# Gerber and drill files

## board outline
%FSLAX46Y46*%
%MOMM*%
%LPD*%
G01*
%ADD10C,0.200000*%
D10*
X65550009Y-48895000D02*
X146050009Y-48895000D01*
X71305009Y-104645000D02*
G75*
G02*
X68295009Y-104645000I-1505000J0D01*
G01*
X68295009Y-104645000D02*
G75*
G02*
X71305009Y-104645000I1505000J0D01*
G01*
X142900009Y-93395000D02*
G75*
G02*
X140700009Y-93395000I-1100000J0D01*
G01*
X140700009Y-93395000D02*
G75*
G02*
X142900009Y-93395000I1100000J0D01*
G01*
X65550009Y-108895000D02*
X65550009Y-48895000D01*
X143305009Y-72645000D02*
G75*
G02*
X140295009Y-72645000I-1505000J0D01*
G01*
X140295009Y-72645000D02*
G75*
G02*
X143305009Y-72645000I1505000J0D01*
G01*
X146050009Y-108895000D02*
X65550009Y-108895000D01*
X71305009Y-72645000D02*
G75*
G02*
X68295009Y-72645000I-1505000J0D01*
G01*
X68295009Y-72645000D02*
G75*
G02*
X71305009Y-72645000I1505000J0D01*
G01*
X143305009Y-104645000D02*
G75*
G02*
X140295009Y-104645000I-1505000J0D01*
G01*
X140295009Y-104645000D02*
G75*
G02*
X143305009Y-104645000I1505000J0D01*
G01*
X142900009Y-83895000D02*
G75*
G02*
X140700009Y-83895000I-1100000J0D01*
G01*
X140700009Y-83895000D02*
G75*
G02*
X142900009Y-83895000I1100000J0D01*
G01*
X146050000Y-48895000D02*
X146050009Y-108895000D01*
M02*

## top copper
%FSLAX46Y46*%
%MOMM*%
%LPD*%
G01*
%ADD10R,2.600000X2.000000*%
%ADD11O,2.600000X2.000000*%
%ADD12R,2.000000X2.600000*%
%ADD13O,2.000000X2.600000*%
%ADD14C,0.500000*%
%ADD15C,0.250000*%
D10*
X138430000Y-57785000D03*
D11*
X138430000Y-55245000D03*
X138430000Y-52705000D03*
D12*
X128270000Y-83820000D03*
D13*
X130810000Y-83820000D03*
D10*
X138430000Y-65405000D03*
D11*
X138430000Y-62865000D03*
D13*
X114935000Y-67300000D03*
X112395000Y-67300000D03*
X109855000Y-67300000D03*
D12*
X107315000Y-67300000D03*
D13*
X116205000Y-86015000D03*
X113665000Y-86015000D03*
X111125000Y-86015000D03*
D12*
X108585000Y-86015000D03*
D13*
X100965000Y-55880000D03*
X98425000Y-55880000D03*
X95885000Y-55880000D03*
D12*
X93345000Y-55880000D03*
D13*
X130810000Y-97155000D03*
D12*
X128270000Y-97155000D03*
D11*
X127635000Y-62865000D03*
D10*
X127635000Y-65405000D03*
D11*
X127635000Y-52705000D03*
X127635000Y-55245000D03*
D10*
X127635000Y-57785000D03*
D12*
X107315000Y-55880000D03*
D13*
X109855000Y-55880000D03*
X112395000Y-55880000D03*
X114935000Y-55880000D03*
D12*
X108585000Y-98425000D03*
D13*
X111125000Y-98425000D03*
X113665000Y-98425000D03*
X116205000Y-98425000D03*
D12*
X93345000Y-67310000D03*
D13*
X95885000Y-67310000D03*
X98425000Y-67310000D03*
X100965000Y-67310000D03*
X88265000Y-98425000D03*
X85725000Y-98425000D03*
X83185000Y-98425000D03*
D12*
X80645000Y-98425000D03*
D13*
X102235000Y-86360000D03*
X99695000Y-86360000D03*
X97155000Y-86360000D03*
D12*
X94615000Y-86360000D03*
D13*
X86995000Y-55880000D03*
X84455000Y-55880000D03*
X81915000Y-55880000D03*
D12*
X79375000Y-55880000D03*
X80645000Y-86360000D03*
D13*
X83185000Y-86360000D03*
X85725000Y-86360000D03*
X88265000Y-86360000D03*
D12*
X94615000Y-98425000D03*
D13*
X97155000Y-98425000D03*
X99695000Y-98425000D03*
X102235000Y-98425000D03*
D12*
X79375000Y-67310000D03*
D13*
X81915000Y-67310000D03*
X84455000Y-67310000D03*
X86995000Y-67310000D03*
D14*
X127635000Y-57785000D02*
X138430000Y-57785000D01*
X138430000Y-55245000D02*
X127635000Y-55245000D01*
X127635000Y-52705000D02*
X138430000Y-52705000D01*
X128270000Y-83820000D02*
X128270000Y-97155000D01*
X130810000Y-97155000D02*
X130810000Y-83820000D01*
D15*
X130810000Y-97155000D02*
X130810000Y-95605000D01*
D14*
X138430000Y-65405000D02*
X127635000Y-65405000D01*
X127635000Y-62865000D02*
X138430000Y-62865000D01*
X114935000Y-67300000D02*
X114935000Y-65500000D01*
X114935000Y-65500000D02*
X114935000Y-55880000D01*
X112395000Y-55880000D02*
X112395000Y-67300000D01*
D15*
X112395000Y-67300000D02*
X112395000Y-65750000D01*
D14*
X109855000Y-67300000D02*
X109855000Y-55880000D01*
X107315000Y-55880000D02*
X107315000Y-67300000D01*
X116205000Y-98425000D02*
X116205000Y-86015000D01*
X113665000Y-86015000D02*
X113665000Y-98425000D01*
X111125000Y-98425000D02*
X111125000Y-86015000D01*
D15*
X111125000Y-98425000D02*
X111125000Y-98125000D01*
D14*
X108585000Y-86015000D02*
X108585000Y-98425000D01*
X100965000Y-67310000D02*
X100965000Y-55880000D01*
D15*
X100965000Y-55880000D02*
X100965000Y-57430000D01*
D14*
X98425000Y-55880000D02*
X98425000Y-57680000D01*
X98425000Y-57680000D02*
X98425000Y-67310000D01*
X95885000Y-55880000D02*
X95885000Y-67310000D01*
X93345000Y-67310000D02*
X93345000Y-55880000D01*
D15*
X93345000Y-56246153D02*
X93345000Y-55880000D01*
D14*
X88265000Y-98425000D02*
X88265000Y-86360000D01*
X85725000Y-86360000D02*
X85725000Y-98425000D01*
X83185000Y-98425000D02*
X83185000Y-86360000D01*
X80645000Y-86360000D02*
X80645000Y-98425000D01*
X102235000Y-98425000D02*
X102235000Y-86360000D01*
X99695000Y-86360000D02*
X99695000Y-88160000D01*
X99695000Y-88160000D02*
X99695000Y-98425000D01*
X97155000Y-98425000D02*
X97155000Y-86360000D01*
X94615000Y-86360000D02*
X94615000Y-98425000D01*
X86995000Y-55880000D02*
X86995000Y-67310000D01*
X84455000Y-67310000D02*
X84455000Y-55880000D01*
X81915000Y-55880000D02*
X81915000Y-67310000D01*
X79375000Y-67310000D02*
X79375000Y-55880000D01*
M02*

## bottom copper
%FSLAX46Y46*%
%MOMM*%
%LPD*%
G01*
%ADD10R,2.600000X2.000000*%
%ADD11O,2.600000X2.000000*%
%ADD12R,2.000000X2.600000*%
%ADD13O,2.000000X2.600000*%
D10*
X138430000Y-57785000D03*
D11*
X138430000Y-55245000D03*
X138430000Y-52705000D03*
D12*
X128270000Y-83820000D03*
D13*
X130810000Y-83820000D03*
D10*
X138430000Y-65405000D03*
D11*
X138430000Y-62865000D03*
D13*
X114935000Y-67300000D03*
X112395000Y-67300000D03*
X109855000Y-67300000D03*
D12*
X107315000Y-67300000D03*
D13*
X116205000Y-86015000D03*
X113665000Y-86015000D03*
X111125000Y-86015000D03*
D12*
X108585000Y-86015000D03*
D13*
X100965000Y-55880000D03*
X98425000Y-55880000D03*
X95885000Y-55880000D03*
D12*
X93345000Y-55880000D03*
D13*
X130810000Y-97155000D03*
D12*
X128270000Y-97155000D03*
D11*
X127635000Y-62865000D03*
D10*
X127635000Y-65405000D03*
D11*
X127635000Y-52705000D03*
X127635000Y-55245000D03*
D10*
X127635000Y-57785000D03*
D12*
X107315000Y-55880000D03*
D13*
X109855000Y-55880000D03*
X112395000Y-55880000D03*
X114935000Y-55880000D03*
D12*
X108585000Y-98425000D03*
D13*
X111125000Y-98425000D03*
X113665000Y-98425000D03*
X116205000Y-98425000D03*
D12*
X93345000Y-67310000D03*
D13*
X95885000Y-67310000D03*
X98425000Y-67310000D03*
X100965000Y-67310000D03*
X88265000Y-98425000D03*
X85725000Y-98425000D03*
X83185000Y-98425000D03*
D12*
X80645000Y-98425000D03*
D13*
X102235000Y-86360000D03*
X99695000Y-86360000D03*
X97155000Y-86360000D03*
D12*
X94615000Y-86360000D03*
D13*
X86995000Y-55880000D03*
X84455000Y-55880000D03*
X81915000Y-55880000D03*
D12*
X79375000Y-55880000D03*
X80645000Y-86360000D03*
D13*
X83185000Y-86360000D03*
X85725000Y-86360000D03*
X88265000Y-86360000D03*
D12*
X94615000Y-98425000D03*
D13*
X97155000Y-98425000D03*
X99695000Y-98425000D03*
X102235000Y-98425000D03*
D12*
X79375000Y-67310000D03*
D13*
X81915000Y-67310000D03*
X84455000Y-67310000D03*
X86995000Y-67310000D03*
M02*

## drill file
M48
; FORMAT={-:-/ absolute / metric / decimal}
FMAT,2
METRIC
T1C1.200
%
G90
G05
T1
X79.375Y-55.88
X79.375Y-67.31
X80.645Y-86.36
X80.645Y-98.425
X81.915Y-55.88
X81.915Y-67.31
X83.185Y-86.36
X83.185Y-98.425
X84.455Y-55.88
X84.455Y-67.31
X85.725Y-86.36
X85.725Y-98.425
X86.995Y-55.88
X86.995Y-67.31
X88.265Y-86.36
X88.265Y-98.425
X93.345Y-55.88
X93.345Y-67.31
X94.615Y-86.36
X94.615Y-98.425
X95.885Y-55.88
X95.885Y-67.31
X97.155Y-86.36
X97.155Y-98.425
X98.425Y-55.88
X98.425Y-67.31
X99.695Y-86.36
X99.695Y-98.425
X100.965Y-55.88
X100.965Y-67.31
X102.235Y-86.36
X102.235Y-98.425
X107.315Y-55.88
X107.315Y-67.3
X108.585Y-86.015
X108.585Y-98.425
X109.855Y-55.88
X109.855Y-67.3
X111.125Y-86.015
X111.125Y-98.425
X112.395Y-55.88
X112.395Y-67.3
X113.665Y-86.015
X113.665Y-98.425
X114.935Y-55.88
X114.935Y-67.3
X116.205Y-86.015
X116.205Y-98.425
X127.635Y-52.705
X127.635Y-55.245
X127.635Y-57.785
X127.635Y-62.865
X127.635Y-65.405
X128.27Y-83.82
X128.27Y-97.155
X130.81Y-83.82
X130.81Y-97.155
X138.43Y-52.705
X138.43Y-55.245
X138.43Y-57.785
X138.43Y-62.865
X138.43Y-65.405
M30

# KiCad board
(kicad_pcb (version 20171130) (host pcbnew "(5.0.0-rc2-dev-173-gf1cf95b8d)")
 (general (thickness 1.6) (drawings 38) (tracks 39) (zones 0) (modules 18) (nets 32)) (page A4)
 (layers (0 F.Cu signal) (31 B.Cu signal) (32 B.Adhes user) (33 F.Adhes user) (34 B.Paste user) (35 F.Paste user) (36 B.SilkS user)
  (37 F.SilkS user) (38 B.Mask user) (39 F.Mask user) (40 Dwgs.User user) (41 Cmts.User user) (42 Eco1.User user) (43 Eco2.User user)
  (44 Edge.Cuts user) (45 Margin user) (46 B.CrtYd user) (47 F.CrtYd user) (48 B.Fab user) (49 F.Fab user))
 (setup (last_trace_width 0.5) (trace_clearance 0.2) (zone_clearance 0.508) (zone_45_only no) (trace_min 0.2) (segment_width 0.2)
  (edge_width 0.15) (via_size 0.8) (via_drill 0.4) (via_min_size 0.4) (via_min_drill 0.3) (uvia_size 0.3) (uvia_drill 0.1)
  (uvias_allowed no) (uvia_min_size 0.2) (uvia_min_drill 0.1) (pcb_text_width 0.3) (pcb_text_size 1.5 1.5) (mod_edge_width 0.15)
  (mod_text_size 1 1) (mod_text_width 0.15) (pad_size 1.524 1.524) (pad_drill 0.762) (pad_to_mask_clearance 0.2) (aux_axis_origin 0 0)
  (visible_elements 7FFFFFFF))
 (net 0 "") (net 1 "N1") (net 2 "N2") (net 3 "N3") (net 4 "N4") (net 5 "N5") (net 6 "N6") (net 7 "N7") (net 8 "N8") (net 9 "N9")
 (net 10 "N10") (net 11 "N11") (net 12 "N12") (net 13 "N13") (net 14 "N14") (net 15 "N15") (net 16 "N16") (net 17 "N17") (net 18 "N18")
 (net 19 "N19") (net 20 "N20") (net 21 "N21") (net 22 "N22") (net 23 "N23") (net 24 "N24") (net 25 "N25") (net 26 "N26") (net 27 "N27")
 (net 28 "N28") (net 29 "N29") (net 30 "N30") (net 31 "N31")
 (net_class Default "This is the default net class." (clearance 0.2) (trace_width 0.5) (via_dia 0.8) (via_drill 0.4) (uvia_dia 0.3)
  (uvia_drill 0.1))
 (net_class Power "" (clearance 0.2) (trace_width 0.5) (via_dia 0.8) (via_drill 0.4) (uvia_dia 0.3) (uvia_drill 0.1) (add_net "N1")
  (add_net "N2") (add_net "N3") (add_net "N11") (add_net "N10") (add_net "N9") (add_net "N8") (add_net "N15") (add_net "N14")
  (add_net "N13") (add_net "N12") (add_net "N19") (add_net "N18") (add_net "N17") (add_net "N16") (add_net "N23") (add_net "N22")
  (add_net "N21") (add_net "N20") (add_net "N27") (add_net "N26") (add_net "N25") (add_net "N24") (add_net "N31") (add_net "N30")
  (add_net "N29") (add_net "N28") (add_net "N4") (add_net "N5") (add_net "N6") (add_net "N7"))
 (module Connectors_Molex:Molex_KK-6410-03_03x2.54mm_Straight (layer F.Cu) (at 138.43 57.785 90)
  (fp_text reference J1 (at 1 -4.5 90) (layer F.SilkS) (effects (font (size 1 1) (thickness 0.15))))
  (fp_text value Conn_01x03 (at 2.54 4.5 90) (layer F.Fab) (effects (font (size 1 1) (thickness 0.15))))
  (pad 1 thru_hole rect (at 0 0 90) (size 2 2.6) (drill 1.2) (layers *.Cu *.Mask) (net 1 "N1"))
  (pad 2 thru_hole oval (at 2.54 0 90) (size 2 2.6) (drill 1.2) (layers *.Cu *.Mask) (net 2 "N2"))
  (pad 3 thru_hole oval (at 5.08 0 90) (size 2 2.6) (drill 1.2) (layers *.Cu *.Mask) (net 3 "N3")))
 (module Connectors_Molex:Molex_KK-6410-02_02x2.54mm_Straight (layer F.Cu) (at 128.27 83.82)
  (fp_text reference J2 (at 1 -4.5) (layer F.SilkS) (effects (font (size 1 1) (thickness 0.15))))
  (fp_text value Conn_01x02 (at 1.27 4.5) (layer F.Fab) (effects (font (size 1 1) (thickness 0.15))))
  (pad 1 thru_hole rect (at 0 0) (size 2 2.6) (drill 1.2) (layers *.Cu *.Mask) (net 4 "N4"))
  (pad 2 thru_hole oval (at 2.54 0) (size 2 2.6) (drill 1.2) (layers *.Cu *.Mask) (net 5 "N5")))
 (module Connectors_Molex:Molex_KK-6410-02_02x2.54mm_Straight (layer F.Cu) (at 138.43 65.405 90)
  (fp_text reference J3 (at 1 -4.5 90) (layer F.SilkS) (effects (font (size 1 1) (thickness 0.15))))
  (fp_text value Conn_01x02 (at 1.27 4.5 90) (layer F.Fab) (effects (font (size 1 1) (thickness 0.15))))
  (pad 1 thru_hole rect (at 0 0 90) (size 2 2.6) (drill 1.2) (layers *.Cu *.Mask) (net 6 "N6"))
  (pad 2 thru_hole oval (at 2.54 0 90) (size 2 2.6) (drill 1.2) (layers *.Cu *.Mask) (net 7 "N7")))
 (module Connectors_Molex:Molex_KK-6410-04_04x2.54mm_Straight (layer F.Cu) (at 107.315 67.3)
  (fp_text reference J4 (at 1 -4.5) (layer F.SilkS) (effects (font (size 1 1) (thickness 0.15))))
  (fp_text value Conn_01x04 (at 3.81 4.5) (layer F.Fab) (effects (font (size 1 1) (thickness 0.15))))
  (pad 4 thru_hole oval (at 7.62 0) (size 2 2.6) (drill 1.2) (layers *.Cu *.Mask) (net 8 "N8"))
  (pad 3 thru_hole oval (at 5.08 0) (size 2 2.6) (drill 1.2) (layers *.Cu *.Mask) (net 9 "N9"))
  (pad 2 thru_hole oval (at 2.54 0) (size 2 2.6) (drill 1.2) (layers *.Cu *.Mask) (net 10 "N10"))
  (pad 1 thru_hole rect (at 0 0) (size 2 2.6) (drill 1.2) (layers *.Cu *.Mask) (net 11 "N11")))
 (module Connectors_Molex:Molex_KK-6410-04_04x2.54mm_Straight (layer F.Cu) (at 108.585 86.015)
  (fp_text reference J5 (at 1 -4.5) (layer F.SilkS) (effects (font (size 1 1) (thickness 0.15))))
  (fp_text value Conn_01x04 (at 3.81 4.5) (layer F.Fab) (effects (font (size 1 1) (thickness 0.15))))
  (pad 4 thru_hole oval (at 7.62 0) (size 2 2.6) (drill 1.2) (layers *.Cu *.Mask) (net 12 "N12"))
  (pad 3 thru_hole oval (at 5.08 0) (size 2 2.6) (drill 1.2) (layers *.Cu *.Mask) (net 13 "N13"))
  (pad 2 thru_hole oval (at 2.54 0) (size 2 2.6) (drill 1.2) (layers *.Cu *.Mask) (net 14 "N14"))
  (pad 1 thru_hole rect (at 0 0) (size 2 2.6) (drill 1.2) (layers *.Cu *.Mask) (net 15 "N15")))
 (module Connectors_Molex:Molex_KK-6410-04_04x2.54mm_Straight (layer F.Cu) (at 93.345 55.88)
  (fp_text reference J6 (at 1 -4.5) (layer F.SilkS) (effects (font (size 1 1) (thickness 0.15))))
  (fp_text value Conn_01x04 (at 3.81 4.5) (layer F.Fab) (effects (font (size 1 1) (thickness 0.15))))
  (pad 4 thru_hole oval (at 7.62 0) (size 2 2.6) (drill 1.2) (layers *.Cu *.Mask) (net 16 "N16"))
  (pad 3 thru_hole oval (at 5.08 0) (size 2 2.6) (drill 1.2) (layers *.Cu *.Mask) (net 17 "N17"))
  (pad 2 thru_hole oval (at 2.54 0) (size 2 2.6) (drill 1.2) (layers *.Cu *.Mask) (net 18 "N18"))
  (pad 1 thru_hole rect (at 0 0) (size 2 2.6) (drill 1.2) (layers *.Cu *.Mask) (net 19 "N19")))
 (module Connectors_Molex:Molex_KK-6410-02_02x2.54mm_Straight (layer F.Cu) (at 128.27 97.155)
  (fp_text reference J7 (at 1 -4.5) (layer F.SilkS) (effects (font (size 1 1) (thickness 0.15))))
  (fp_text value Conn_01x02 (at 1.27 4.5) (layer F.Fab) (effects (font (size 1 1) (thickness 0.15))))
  (pad 2 thru_hole oval (at 2.54 0) (size 2 2.6) (drill 1.2) (layers *.Cu *.Mask) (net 5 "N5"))
  (pad 1 thru_hole rect (at 0 0) (size 2 2.6) (drill 1.2) (layers *.Cu *.Mask) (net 4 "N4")))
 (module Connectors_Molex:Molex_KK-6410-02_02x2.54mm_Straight (layer F.Cu) (at 127.635 65.405 90)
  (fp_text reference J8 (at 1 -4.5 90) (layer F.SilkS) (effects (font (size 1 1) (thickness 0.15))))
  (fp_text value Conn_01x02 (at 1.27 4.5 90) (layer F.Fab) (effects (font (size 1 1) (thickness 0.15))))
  (pad 2 thru_hole oval (at 2.54 0 90) (size 2 2.6) (drill 1.2) (layers *.Cu *.Mask) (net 7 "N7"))
  (pad 1 thru_hole rect (at 0 0 90) (size 2 2.6) (drill 1.2) (layers *.Cu *.Mask) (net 6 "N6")))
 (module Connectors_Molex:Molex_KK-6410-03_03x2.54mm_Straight (layer F.Cu) (at 127.635 57.785 90)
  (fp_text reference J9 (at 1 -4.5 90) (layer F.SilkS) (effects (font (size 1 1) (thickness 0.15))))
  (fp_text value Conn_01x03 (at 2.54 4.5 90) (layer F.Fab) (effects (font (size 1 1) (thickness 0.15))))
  (pad 3 thru_hole oval (at 5.08 0 90) (size 2 2.6) (drill 1.2) (layers *.Cu *.Mask) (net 3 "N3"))
  (pad 2 thru_hole oval (at 2.54 0 90) (size 2 2.6) (drill 1.2) (layers *.Cu *.Mask) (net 2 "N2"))
  (pad 1 thru_hole rect (at 0 0 90) (size 2 2.6) (drill 1.2) (layers *.Cu *.Mask) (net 1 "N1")))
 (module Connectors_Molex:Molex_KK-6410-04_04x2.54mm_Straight (layer F.Cu) (at 107.315 55.88)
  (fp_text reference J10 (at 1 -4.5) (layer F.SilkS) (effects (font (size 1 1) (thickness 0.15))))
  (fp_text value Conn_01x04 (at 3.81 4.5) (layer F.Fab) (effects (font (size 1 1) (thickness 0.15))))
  (pad 1 thru_hole rect (at 0 0) (size 2 2.6) (drill 1.2) (layers *.Cu *.Mask) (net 11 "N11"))
  (pad 2 thru_hole oval (at 2.54 0) (size 2 2.6) (drill 1.2) (layers *.Cu *.Mask) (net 10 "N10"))
  (pad 3 thru_hole oval (at 5.08 0) (size 2 2.6) (drill 1.2) (layers *.Cu *.Mask) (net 9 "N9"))
  (pad 4 thru_hole oval (at 7.62 0) (size 2 2.6) (drill 1.2) (layers *.Cu *.Mask) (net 8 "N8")))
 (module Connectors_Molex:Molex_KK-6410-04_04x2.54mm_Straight (layer F.Cu) (at 108.585 98.425)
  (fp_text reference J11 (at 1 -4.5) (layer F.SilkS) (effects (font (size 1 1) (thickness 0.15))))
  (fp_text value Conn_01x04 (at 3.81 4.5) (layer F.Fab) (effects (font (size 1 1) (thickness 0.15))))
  (pad 1 thru_hole rect (at 0 0) (size 2 2.6) (drill 1.2) (layers *.Cu *.Mask) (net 15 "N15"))
  (pad 2 thru_hole oval (at 2.54 0) (size 2 2.6) (drill 1.2) (layers *.Cu *.Mask) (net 14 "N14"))
  (pad 3 thru_hole oval (at 5.08 0) (size 2 2.6) (drill 1.2) (layers *.Cu *.Mask) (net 13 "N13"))
  (pad 4 thru_hole oval (at 7.62 0) (size 2 2.6) (drill 1.2) (layers *.Cu *.Mask) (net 12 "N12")))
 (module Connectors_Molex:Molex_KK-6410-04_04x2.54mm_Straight (layer F.Cu) (at 93.345 67.31)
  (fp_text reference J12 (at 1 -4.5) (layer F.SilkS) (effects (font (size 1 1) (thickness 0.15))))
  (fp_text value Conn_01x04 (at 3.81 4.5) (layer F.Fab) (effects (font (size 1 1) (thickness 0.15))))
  (pad 1 thru_hole rect (at 0 0) (size 2 2.6) (drill 1.2) (layers *.Cu *.Mask) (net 19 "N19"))
  (pad 2 thru_hole oval (at 2.54 0) (size 2 2.6) (drill 1.2) (layers *.Cu *.Mask) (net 18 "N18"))
  (pad 3 thru_hole oval (at 5.08 0) (size 2 2.6) (drill 1.2) (layers *.Cu *.Mask) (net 17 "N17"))
  (pad 4 thru_hole oval (at 7.62 0) (size 2 2.6) (drill 1.2) (layers *.Cu *.Mask) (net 16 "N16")))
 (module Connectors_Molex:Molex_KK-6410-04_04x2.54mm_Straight (layer F.Cu) (at 80.645 98.425)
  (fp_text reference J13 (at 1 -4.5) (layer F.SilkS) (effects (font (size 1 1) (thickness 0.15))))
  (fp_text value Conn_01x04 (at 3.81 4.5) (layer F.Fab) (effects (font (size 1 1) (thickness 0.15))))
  (pad 4 thru_hole oval (at 7.62 0) (size 2 2.6) (drill 1.2) (layers *.Cu *.Mask) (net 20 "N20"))
  (pad 3 thru_hole oval (at 5.08 0) (size 2 2.6) (drill 1.2) (layers *.Cu *.Mask) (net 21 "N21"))
  (pad 2 thru_hole oval (at 2.54 0) (size 2 2.6) (drill 1.2) (layers *.Cu *.Mask) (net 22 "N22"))
  (pad 1 thru_hole rect (at 0 0) (size 2 2.6) (drill 1.2) (layers *.Cu *.Mask) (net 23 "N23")))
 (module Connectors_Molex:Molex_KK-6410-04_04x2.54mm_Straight (layer F.Cu) (at 94.615 86.36)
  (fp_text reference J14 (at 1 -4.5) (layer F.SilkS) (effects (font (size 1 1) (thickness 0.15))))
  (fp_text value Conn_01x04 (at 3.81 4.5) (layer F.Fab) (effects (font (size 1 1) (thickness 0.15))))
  (pad 4 thru_hole oval (at 7.62 0) (size 2 2.6) (drill 1.2) (layers *.Cu *.Mask) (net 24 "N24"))
  (pad 3 thru_hole oval (at 5.08 0) (size 2 2.6) (drill 1.2) (layers *.Cu *.Mask) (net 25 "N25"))
  (pad 2 thru_hole oval (at 2.54 0) (size 2 2.6) (drill 1.2) (layers *.Cu *.Mask) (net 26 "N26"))
  (pad 1 thru_hole rect (at 0 0) (size 2 2.6) (drill 1.2) (layers *.Cu *.Mask) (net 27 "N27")))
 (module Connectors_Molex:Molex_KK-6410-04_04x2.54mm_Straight (layer F.Cu) (at 79.375 55.88)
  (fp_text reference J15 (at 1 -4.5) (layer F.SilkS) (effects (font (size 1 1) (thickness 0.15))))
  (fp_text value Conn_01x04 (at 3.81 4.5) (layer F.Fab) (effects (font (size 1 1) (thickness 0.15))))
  (pad 4 thru_hole oval (at 7.62 0) (size 2 2.6) (drill 1.2) (layers *.Cu *.Mask) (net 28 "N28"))
  (pad 3 thru_hole oval (at 5.08 0) (size 2 2.6) (drill 1.2) (layers *.Cu *.Mask) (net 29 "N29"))
  (pad 2 thru_hole oval (at 2.54 0) (size 2 2.6) (drill 1.2) (layers *.Cu *.Mask) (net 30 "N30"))
  (pad 1 thru_hole rect (at 0 0) (size 2 2.6) (drill 1.2) (layers *.Cu *.Mask) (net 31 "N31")))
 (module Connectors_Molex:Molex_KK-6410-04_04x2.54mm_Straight (layer F.Cu) (at 80.645 86.36)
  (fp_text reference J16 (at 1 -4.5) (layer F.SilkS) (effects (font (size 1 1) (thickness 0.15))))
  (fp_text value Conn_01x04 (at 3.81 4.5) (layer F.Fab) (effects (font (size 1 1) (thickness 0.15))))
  (pad 1 thru_hole rect (at 0 0) (size 2 2.6) (drill 1.2) (layers *.Cu *.Mask) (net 23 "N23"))
  (pad 2 thru_hole oval (at 2.54 0) (size 2 2.6) (drill 1.2) (layers *.Cu *.Mask) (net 22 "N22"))
  (pad 3 thru_hole oval (at 5.08 0) (size 2 2.6) (drill 1.2) (layers *.Cu *.Mask) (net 21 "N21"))
  (pad 4 thru_hole oval (at 7.62 0) (size 2 2.6) (drill 1.2) (layers *.Cu *.Mask) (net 20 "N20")))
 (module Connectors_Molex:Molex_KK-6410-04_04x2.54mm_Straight (layer F.Cu) (at 94.615 98.425)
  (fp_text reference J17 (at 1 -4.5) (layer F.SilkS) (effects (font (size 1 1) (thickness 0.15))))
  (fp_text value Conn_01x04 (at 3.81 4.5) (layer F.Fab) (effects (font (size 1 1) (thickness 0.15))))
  (pad 1 thru_hole rect (at 0 0) (size 2 2.6) (drill 1.2) (layers *.Cu *.Mask) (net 27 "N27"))
  (pad 2 thru_hole oval (at 2.54 0) (size 2 2.6) (drill 1.2) (layers *.Cu *.Mask) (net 26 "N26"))
  (pad 3 thru_hole oval (at 5.08 0) (size 2 2.6) (drill 1.2) (layers *.Cu *.Mask) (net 25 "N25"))
  (pad 4 thru_hole oval (at 7.62 0) (size 2 2.6) (drill 1.2) (layers *.Cu *.Mask) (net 24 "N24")))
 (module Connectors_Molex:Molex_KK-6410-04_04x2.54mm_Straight (layer F.Cu) (at 79.375 67.31)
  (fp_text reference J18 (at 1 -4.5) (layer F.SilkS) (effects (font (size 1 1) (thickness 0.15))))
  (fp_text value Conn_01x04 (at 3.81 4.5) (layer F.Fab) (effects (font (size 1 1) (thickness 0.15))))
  (pad 1 thru_hole rect (at 0 0) (size 2 2.6) (drill 1.2) (layers *.Cu *.Mask) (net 31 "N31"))
  (pad 2 thru_hole oval (at 2.54 0) (size 2 2.6) (drill 1.2) (layers *.Cu *.Mask) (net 30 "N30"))
  (pad 3 thru_hole oval (at 5.08 0) (size 2 2.6) (drill 1.2) (layers *.Cu *.Mask) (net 29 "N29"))
  (pad 4 thru_hole oval (at 7.62 0) (size 2 2.6) (drill 1.2) (layers *.Cu *.Mask) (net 28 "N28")))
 (gr_line (start 65.550009 48.895) (end 146.050009 48.895) (layer Edge.Cuts) (width 0.2))
 (gr_circle (center 69.800009 104.645) (end 71.305009 104.645) (layer Edge.Cuts) (width 0.2))
 (gr_circle (center 141.800009 93.395) (end 142.900009 93.395) (layer Edge.Cuts) (width 0.2))
 (gr_line (start 65.550009 108.895) (end 65.550009 48.895) (layer Edge.Cuts) (width 0.2))
 (gr_circle (center 141.800009 72.645) (end 143.305009 72.645) (layer Edge.Cuts) (width 0.2))
 (gr_line (start 146.050009 108.895) (end 65.550009 108.895) (layer Edge.Cuts) (width 0.2))
 (gr_circle (center 69.800009 72.645) (end 71.305009 72.645) (layer Edge.Cuts) (width 0.2))
 (gr_circle (center 141.800009 104.645) (end 143.305009 104.645) (layer Edge.Cuts) (width 0.2))
 (gr_circle (center 141.800009 83.895) (end 142.900009 83.895) (layer Edge.Cuts) (width 0.2))
 (gr_line (start 146.05 48.895) (end 146.050009 108.895) (layer Edge.Cuts) (width 0.2))
 (segment (start 127.635 57.785) (end 138.43 57.785) (width 0.5) (layer F.Cu) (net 1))
 (segment (start 138.43 55.245) (end 127.635 55.245) (width 0.5) (layer F.Cu) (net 2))
 (segment (start 127.635 52.705) (end 138.43 52.705) (width 0.5) (layer F.Cu) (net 3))
 (segment (start 128.27 83.82) (end 128.27 97.155) (width 0.5) (layer F.Cu) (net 4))
 (segment (start 130.81 97.155) (end 130.81 83.82) (width 0.5) (layer F.Cu) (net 5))
 (segment (start 130.81 97.155) (end 130.81 95.605) (width 0.25) (layer F.Cu) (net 5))
 (segment (start 138.43 65.405) (end 127.635 65.405) (width 0.5) (layer F.Cu) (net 6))
 (segment (start 127.635 62.865) (end 138.43 62.865) (width 0.5) (layer F.Cu) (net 7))
 (segment (start 114.935 67.3) (end 114.935 65.5) (width 0.5) (layer F.Cu) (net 8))
 (segment (start 114.935 65.5) (end 114.935 55.88) (width 0.5) (layer F.Cu) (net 8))
 (segment (start 112.395 55.88) (end 112.395 67.3) (width 0.5) (layer F.Cu) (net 9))
 (segment (start 112.395 67.3) (end 112.395 65.75) (width 0.25) (layer F.Cu) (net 9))
 (segment (start 109.855 67.3) (end 109.855 55.88) (width 0.5) (layer F.Cu) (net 10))
 (segment (start 107.315 55.88) (end 107.315 67.3) (width 0.5) (layer F.Cu) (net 11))
 (segment (start 116.205 98.425) (end 116.205 86.015) (width 0.5) (layer F.Cu) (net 12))
 (segment (start 113.665 86.015) (end 113.665 98.425) (width 0.5) (layer F.Cu) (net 13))
 (segment (start 111.125 98.425) (end 111.125 86.015) (width 0.5) (layer F.Cu) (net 14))
 (segment (start 111.125 98.425) (end 111.125 98.125) (width 0.25) (layer F.Cu) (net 14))
 (segment (start 108.585 86.015) (end 108.585 98.425) (width 0.5) (layer F.Cu) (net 15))
 (segment (start 100.965 67.31) (end 100.965 55.88) (width 0.5) (layer F.Cu) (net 16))
 (segment (start 100.965 55.88) (end 100.965 57.43) (width 0.25) (layer F.Cu) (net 16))
 (segment (start 98.425 55.88) (end 98.425 57.68) (width 0.5) (layer F.Cu) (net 17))
 (segment (start 98.425 57.68) (end 98.425 67.31) (width 0.5) (layer F.Cu) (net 17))
 (segment (start 95.885 55.88) (end 95.885 67.31) (width 0.5) (layer F.Cu) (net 18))
 (segment (start 93.345 67.31) (end 93.345 55.88) (width 0.5) (layer F.Cu) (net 19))
 (segment (start 93.345 56.246153) (end 93.345 55.88) (width 0.25) (layer F.Cu) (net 19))
 (segment (start 88.265 98.425) (end 88.265 86.36) (width 0.5) (layer F.Cu) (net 20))
 (segment (start 85.725 86.36) (end 85.725 98.425) (width 0.5) (layer F.Cu) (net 21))
 (segment (start 83.185 98.425) (end 83.185 86.36) (width 0.5) (layer F.Cu) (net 22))
 (segment (start 80.645 86.36) (end 80.645 98.425) (width 0.5) (layer F.Cu) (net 23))
 (segment (start 102.235 98.425) (end 102.235 86.36) (width 0.5) (layer F.Cu) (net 24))
 (segment (start 99.695 86.36) (end 99.695 88.16) (width 0.5) (layer F.Cu) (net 25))
 (segment (start 99.695 88.16) (end 99.695 98.425) (width 0.5) (layer F.Cu) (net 25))
 (segment (start 97.155 98.425) (end 97.155 86.36) (width 0.5) (layer F.Cu) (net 26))
 (segment (start 94.615 86.36) (end 94.615 98.425) (width 0.5) (layer F.Cu) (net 27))
 (segment (start 86.995 55.88) (end 86.995 67.31) (width 0.5) (layer F.Cu) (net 28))
 (segment (start 84.455 67.31) (end 84.455 55.88) (width 0.5) (layer F.Cu) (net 29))
 (segment (start 81.915 55.88) (end 81.915 67.31) (width 0.5) (layer F.Cu) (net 30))
 (segment (start 79.375 67.31) (end 79.375 55.88) (width 0.5) (layer F.Cu) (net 31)))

